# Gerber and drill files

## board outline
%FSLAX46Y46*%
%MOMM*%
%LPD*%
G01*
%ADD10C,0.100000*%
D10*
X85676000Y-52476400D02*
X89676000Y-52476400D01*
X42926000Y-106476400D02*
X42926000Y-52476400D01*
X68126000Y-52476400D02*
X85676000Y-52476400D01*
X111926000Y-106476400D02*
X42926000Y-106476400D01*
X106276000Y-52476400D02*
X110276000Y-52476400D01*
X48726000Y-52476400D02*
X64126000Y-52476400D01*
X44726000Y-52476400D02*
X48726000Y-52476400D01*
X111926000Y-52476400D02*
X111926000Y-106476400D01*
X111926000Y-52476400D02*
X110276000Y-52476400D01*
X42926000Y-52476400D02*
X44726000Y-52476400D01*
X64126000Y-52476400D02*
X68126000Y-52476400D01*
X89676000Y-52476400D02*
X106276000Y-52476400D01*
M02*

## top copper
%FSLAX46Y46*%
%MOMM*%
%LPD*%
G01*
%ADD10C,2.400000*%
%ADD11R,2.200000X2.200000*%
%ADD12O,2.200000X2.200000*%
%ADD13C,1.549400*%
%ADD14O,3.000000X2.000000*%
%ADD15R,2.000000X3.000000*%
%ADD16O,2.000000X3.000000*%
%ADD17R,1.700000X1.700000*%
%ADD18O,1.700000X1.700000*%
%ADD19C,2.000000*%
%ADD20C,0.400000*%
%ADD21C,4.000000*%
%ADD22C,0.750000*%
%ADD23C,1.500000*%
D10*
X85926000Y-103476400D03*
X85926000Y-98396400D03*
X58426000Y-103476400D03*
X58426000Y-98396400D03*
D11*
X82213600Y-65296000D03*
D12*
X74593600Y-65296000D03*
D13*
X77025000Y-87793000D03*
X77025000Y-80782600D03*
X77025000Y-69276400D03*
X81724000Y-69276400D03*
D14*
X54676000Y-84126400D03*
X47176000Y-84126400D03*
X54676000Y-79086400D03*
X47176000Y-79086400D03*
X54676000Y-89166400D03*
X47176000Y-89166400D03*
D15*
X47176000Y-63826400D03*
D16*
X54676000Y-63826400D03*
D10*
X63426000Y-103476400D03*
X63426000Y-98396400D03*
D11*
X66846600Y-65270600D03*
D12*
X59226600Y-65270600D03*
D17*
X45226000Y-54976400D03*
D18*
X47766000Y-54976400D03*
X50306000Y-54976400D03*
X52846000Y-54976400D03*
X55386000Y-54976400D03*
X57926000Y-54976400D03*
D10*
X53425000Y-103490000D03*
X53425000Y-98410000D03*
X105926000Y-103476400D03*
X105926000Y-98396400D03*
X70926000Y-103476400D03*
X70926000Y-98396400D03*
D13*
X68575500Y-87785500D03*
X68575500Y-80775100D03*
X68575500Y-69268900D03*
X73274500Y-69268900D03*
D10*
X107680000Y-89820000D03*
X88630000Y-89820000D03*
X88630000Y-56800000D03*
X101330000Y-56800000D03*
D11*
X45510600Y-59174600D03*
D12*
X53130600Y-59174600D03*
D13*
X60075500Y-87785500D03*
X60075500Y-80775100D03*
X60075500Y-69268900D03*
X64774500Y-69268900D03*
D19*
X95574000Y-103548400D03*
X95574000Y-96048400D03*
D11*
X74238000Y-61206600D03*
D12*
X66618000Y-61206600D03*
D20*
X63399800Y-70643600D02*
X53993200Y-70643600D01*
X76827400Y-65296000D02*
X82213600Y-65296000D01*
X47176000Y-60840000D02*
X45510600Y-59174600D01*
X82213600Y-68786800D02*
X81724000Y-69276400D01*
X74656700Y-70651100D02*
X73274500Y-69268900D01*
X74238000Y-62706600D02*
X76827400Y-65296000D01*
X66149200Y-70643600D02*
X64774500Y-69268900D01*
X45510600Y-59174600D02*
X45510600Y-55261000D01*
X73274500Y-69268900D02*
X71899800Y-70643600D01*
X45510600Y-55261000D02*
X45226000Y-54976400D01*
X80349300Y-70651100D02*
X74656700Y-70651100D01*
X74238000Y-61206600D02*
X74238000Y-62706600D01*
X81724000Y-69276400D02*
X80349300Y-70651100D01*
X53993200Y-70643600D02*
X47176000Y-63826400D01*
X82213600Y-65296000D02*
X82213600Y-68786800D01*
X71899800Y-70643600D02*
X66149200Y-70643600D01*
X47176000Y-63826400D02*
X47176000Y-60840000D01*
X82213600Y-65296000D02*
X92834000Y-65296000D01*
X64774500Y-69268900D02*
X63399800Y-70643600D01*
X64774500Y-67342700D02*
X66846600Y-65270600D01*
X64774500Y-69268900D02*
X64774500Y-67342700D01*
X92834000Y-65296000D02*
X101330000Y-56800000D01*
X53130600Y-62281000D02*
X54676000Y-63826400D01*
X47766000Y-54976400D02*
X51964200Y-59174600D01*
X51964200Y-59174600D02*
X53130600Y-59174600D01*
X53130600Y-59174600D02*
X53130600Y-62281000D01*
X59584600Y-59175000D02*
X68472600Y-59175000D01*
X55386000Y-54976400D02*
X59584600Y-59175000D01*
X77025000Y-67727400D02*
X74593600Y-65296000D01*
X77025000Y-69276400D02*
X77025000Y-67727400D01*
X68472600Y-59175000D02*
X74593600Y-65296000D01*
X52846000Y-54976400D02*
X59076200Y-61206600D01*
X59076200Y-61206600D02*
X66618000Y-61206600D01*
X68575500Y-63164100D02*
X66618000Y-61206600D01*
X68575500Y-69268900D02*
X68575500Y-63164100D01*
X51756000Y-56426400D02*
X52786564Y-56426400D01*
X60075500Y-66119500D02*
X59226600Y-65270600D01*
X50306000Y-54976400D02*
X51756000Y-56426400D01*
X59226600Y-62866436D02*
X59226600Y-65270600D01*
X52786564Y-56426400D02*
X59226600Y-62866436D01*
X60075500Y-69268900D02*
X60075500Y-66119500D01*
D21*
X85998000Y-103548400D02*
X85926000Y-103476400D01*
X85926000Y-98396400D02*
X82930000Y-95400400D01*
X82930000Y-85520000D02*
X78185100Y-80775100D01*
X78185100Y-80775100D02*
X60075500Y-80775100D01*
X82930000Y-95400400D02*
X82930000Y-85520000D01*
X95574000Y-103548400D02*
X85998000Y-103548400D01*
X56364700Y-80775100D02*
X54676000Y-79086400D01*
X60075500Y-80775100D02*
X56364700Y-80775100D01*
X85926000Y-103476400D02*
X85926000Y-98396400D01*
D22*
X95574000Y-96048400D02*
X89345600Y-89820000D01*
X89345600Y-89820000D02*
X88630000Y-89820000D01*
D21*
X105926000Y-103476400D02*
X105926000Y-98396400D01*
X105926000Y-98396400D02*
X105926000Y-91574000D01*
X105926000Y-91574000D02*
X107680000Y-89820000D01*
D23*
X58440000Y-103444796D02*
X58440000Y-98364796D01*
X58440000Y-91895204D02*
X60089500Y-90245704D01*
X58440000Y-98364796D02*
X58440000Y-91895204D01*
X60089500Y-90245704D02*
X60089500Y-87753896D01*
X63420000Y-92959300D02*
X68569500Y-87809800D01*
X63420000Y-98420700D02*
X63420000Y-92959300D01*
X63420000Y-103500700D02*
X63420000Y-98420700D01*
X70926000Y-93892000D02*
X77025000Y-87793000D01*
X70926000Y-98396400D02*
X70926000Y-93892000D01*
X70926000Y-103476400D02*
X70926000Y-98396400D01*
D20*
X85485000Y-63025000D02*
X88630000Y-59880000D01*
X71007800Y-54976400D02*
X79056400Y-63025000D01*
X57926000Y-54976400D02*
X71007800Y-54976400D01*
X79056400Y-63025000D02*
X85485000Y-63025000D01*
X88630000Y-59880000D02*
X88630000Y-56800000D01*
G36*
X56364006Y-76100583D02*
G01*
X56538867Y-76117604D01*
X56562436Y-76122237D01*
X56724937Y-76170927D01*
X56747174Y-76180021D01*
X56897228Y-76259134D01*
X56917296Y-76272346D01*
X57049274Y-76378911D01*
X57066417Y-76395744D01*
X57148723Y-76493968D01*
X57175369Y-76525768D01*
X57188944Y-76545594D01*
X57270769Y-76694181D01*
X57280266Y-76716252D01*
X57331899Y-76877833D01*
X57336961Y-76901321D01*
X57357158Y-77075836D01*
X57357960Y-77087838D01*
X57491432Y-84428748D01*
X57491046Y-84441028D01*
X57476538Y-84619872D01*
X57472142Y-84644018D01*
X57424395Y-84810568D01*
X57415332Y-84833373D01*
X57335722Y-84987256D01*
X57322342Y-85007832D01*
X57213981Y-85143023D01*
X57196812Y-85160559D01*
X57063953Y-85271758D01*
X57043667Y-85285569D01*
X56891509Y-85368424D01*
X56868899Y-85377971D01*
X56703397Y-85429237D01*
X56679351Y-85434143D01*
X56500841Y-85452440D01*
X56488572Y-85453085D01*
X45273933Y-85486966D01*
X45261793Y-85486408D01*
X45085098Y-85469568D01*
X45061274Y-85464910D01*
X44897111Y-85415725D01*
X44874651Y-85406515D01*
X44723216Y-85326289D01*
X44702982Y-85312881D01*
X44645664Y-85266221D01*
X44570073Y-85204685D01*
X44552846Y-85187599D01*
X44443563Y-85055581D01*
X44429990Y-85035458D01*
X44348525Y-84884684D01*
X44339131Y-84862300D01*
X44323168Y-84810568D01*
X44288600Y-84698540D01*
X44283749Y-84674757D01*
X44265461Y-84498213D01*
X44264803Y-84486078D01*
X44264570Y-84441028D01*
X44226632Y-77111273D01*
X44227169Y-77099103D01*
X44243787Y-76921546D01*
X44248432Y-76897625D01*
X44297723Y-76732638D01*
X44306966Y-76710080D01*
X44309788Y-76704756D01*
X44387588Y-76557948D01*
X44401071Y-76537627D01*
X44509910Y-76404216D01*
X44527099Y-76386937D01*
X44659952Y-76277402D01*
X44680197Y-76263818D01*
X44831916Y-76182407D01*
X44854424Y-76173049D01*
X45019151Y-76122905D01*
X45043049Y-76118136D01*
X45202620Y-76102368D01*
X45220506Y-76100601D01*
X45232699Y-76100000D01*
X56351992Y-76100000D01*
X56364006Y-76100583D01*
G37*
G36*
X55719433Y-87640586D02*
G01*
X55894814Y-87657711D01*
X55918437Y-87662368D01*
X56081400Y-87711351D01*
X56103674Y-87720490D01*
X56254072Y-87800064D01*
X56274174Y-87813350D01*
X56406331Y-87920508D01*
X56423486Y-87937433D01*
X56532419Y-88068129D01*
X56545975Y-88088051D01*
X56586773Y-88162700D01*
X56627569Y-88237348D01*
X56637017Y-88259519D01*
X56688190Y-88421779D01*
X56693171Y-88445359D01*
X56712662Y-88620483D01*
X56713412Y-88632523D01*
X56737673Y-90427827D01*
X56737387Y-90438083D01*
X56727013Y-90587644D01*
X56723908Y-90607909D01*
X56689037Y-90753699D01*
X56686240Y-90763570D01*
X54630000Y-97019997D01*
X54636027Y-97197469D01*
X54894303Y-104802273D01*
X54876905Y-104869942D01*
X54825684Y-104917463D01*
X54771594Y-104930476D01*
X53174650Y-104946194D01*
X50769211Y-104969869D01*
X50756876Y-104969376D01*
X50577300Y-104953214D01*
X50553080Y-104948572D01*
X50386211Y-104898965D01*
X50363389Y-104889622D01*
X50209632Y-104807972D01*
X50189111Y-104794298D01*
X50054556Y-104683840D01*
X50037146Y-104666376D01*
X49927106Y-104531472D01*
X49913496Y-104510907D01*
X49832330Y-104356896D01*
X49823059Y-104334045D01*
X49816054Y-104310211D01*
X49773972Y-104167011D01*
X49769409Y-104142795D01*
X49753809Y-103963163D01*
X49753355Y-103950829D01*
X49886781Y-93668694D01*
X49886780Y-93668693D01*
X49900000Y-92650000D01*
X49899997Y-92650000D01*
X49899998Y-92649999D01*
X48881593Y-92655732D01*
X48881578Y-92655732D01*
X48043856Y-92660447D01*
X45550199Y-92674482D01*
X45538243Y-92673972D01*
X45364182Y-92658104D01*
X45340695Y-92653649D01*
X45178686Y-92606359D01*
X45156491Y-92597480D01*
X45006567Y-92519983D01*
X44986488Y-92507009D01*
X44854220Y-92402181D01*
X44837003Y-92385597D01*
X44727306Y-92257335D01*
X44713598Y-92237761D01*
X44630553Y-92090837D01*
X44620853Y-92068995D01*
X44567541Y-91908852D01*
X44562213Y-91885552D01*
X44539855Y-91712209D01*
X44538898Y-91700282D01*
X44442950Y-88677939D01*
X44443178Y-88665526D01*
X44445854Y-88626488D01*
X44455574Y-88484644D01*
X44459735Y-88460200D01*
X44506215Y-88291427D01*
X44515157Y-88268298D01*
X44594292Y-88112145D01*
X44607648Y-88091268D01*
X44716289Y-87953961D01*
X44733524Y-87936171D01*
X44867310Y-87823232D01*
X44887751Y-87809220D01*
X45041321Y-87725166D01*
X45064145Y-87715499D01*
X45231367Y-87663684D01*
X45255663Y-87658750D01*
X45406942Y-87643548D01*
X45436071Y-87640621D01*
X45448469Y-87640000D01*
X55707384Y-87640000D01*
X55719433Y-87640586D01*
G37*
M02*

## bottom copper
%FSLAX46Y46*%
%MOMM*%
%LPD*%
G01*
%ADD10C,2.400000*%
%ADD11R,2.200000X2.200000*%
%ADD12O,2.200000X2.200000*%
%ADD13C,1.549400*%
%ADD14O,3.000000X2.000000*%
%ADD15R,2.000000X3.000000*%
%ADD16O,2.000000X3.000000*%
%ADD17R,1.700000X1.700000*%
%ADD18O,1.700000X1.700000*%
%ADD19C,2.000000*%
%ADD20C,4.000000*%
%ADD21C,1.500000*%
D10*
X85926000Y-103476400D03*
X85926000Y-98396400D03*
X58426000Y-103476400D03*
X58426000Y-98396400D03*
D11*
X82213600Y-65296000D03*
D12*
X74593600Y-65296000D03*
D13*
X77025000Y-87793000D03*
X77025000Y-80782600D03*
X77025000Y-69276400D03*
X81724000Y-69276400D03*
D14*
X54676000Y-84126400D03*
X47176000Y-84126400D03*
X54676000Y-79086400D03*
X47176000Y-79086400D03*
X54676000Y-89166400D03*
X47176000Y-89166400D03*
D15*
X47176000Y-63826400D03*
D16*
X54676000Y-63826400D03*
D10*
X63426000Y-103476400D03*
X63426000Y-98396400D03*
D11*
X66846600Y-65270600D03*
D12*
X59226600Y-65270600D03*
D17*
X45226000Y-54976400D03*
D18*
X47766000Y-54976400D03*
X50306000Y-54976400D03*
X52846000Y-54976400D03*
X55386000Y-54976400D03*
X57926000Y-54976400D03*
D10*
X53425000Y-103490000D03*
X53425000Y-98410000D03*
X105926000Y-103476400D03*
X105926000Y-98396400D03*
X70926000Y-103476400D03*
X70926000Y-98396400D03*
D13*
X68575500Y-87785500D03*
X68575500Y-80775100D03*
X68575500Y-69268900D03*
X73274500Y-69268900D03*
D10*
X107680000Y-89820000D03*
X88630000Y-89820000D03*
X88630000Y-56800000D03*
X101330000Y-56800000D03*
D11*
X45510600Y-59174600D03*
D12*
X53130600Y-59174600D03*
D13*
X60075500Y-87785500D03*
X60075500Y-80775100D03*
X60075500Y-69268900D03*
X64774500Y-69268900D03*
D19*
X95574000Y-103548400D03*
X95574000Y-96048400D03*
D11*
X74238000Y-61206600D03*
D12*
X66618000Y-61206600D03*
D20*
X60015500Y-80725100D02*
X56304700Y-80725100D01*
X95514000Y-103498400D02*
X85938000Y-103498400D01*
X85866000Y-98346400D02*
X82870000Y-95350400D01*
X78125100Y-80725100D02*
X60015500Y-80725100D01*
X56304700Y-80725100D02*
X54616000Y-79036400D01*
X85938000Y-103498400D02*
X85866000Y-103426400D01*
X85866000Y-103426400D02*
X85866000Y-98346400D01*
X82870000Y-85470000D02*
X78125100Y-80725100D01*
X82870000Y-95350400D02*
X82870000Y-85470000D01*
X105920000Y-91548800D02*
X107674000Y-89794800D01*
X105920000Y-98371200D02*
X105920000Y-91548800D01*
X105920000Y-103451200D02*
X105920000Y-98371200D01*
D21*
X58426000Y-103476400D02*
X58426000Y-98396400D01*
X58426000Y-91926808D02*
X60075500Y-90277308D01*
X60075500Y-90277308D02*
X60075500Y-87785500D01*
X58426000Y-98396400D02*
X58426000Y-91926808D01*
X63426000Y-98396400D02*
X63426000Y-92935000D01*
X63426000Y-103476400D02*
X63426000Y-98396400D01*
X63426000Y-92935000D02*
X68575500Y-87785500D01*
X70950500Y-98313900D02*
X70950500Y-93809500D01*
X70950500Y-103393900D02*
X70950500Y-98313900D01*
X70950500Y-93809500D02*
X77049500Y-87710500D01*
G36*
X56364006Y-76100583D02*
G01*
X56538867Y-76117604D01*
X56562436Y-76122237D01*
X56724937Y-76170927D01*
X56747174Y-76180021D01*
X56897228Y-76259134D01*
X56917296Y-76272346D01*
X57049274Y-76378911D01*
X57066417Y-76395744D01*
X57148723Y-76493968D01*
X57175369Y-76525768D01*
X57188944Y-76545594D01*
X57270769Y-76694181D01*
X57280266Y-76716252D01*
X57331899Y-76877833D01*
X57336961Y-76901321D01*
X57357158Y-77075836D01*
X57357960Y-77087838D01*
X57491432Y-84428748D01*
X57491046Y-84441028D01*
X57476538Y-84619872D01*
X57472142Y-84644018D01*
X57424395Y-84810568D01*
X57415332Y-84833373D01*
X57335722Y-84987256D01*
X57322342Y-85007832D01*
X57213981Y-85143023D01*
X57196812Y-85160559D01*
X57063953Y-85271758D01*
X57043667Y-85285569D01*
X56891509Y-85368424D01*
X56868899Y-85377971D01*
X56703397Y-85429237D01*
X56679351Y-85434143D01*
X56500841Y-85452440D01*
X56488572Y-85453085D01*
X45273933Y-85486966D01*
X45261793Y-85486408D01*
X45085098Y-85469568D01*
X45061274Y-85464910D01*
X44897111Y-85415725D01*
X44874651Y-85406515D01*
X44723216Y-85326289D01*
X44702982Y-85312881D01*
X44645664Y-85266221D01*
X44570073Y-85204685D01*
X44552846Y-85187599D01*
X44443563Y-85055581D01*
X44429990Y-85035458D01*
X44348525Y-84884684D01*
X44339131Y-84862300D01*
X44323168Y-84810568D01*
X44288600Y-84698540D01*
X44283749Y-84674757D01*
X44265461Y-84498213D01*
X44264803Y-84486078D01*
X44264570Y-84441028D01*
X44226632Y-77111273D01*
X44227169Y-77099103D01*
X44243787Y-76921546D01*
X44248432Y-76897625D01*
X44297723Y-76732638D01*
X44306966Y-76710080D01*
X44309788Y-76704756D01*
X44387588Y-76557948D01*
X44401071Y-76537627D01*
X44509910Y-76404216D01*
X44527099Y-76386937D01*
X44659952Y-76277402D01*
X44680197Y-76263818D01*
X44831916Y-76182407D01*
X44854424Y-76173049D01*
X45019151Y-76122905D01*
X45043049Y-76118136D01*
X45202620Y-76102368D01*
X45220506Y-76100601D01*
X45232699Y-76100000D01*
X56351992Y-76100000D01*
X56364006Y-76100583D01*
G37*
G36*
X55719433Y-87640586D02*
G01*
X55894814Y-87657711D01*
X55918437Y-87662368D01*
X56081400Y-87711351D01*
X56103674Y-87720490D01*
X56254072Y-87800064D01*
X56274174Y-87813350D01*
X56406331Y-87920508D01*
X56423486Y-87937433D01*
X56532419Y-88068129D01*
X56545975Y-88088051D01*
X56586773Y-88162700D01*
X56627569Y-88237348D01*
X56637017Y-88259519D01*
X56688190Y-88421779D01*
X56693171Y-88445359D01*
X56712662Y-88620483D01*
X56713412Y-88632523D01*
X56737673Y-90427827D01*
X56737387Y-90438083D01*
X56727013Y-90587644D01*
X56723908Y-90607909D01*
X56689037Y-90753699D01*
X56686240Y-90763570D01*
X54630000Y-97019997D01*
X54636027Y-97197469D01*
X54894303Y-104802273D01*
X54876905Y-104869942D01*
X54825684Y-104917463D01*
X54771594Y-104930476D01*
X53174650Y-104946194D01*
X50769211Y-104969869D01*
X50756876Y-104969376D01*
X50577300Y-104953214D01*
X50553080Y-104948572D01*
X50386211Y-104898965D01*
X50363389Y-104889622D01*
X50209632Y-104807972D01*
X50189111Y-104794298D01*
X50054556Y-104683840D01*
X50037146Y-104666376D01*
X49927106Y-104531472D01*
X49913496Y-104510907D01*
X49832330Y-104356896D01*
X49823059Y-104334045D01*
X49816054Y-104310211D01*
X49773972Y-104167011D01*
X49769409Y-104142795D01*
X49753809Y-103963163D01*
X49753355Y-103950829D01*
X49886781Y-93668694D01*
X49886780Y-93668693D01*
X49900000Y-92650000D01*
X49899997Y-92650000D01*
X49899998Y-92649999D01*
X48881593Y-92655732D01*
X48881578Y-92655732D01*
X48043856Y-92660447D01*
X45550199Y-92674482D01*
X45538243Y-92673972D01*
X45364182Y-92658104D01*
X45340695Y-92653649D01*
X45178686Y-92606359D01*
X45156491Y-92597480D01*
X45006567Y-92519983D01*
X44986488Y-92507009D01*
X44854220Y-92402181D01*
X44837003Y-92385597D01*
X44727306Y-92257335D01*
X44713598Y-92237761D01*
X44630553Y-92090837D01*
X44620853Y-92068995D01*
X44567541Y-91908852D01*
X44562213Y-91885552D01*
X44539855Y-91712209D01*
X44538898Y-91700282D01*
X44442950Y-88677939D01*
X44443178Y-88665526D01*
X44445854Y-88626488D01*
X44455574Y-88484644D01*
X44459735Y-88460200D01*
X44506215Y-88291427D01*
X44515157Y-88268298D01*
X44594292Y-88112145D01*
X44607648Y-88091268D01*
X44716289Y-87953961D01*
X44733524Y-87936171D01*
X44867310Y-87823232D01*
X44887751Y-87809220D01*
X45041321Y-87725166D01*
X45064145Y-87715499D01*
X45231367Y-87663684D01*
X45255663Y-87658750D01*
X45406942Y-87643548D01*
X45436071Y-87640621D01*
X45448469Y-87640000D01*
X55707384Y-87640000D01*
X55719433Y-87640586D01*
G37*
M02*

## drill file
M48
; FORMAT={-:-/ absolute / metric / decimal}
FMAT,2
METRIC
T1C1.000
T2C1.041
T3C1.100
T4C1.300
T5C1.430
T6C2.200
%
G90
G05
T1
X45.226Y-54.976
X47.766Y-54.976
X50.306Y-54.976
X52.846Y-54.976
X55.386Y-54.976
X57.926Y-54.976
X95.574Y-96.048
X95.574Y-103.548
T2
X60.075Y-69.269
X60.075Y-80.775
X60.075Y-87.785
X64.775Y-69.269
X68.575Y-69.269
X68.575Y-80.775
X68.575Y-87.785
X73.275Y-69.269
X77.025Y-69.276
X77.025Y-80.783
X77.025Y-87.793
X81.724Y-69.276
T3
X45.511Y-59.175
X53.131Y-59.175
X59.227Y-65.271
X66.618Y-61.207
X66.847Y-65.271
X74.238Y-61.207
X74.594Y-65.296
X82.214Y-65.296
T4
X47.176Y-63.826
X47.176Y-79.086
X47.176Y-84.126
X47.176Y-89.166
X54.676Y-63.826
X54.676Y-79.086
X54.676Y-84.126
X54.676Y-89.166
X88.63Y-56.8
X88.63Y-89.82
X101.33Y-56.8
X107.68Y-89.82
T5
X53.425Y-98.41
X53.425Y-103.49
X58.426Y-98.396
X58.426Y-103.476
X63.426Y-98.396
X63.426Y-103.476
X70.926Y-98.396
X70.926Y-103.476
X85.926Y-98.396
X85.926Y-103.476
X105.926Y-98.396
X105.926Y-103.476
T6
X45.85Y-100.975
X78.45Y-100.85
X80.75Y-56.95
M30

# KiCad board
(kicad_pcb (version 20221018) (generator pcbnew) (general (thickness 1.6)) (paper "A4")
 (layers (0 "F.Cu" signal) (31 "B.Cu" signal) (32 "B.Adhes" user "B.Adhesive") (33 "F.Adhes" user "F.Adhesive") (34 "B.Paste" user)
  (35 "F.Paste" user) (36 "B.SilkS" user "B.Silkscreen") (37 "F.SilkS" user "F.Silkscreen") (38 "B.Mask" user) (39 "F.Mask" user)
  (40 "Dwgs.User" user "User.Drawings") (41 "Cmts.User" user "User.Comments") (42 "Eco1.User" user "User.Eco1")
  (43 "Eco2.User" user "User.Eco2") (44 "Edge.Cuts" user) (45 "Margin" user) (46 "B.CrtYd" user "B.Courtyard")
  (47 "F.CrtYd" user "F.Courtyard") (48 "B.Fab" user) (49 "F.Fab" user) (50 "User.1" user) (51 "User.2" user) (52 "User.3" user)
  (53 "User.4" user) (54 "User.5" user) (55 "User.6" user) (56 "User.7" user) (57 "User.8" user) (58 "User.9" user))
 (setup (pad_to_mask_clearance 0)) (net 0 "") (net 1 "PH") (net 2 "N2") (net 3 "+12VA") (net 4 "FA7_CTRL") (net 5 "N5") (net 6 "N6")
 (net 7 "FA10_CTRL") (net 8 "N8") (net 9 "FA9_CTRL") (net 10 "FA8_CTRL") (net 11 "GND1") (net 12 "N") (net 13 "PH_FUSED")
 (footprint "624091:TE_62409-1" (layer "F.Cu") (at 85.926 100.9364 90)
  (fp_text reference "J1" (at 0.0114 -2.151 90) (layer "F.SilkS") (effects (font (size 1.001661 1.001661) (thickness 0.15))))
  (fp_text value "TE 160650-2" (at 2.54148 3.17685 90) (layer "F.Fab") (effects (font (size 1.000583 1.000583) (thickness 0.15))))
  (pad "1" thru_hole circle (at -2.54 0 90) (size 2.4 2.4) (drill 1.43) (layers "*.Cu" "*.Mask") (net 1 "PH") (solder_mask_margin 0.102))
  (pad "1" thru_hole circle (at 2.54 0 90) (size 2.4 2.4) (drill 1.43) (layers "*.Cu" "*.Mask") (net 1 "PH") (solder_mask_margin 0.102)))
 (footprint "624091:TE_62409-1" (layer "F.Cu") (at 58.426 100.9364 90)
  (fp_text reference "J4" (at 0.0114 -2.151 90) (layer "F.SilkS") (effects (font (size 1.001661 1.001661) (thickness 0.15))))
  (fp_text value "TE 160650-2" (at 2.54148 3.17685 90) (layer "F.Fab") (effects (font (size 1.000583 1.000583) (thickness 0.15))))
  (pad "1" thru_hole circle (at -2.54 0 90) (size 2.4 2.4) (drill 1.43) (layers "*.Cu" "*.Mask") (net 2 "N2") (solder_mask_margin 0.102))
  (pad "1" thru_hole circle (at 2.54 0 90) (size 2.4 2.4) (drill 1.43) (layers "*.Cu" "*.Mask") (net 2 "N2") (solder_mask_margin 0.102)))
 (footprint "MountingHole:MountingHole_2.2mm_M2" (layer "F.Cu") (at 80.75 56.95)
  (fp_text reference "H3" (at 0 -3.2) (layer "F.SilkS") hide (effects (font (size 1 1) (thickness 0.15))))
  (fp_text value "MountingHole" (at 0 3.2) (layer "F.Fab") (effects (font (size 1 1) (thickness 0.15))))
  (pad "" np_thru_hole circle (at 0 0) (size 2.2 2.2) (drill 2.2) (layers "F&B.Cu" "*.Mask")))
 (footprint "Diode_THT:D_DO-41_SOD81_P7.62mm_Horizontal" (layer "F.Cu") (at 82.2136 65.296 180)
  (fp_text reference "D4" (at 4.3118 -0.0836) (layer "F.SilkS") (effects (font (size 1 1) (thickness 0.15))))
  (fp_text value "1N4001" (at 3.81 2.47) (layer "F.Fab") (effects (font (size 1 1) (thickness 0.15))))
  (pad "1" thru_hole rect (at 0 0 180) (size 2.2 2.2) (drill 1.1) (layers "*.Cu" "*.Mask") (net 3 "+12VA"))
  (pad "2" thru_hole oval (at 7.62 0 180) (size 2.2 2.2) (drill 1.1) (layers "*.Cu" "*.Mask") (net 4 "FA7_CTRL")))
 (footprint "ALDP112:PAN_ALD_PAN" (layer "F.Cu") (at 81.725 87.793 180)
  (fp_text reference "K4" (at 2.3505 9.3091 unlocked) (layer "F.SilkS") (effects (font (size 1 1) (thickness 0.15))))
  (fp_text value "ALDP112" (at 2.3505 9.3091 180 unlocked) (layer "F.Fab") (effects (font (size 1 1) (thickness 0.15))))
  (pad "1" thru_hole circle (at 4.7 0 180) (size 1.5494 1.5494) (drill 1.0414) (layers "*.Cu" "*.Mask") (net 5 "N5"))
  (pad "2" thru_hole circle (at 4.7 7.0104 180) (size 1.5494 1.5494) (drill 1.0414) (layers "*.Cu" "*.Mask") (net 1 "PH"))
  (pad "3" thru_hole circle (at 4.7 18.5166 180) (size 1.5494 1.5494) (drill 1.0414) (layers "*.Cu" "*.Mask") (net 4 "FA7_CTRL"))
  (pad "4" thru_hole circle (at 0.001 18.5166 180) (size 1.5494 1.5494) (drill 1.0414) (layers "*.Cu" "*.Mask") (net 3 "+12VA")))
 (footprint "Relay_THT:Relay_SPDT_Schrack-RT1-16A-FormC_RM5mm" (layer "F.Cu") (at 47.176 63.8264 -90)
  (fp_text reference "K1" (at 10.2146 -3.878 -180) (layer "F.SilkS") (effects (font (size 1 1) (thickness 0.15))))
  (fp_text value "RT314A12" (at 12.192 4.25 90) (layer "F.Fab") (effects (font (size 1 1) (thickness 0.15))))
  (pad "11" thru_hole oval (at 20.3 -7.5 90) (size 2 3) (drill 1.3) (layers "*.Cu" "*.Mask") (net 1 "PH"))
  (pad "11" thru_hole oval (at 20.3 0 90) (size 2 3) (drill 1.3) (layers "*.Cu" "*.Mask") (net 1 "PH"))
  (pad "12" thru_hole oval (at 15.26 -7.5 90) (size 2 3) (drill 1.3) (layers "*.Cu" "*.Mask") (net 1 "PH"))
  (pad "12" thru_hole oval (at 15.26 0 90) (size 2 3) (drill 1.3) (layers "*.Cu" "*.Mask") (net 1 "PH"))
  (pad "14" thru_hole oval (at 25.34 -7.5 90) (size 2 3) (drill 1.3) (layers "*.Cu" "*.Mask") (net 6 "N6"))
  (pad "14" thru_hole oval (at 25.34 0 90) (size 2 3) (drill 1.3) (layers "*.Cu" "*.Mask") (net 6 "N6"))
  (pad "A1" thru_hole rect (at 0 0 90) (size 3 2) (drill 1.3) (layers "*.Cu" "*.Mask") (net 3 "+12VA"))
  (pad "A2" thru_hole oval (at 0 -7.5 90) (size 3 2) (drill 1.3) (layers "*.Cu" "*.Mask") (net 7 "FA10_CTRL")))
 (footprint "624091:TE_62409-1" (layer "F.Cu") (at 63.426 100.9364 90)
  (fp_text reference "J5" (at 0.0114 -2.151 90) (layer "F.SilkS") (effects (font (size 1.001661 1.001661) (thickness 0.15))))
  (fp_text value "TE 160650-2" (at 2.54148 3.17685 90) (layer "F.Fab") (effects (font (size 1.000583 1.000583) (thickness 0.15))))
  (pad "1" thru_hole circle (at -2.54 0 90) (size 2.4 2.4) (drill 1.43) (layers "*.Cu" "*.Mask") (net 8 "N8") (solder_mask_margin 0.102))
  (pad "1" thru_hole circle (at 2.54 0 90) (size 2.4 2.4) (drill 1.43) (layers "*.Cu" "*.Mask") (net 8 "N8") (solder_mask_margin 0.102)))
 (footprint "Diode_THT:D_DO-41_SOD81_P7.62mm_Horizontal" (layer "F.Cu") (at 66.8466 65.2706 180)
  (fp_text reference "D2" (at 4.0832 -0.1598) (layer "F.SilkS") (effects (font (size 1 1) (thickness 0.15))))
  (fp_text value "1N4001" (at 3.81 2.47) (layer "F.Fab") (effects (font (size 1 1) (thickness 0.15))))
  (pad "1" thru_hole rect (at 0 0 180) (size 2.2 2.2) (drill 1.1) (layers "*.Cu" "*.Mask") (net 3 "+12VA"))
  (pad "2" thru_hole oval (at 7.62 0 180) (size 2.2 2.2) (drill 1.1) (layers "*.Cu" "*.Mask") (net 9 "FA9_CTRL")))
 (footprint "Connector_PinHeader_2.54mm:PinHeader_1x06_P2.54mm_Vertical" (layer "F.Cu") (at 45.226 54.9764 90)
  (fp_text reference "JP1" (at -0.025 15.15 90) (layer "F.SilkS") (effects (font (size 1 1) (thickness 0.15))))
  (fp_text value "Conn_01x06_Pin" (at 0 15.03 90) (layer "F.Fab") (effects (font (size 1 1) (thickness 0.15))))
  (pad "1" thru_hole rect (at 0 0 90) (size 1.7 1.7) (drill 1) (layers "*.Cu" "*.Mask") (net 3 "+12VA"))
  (pad "2" thru_hole oval (at 0 2.54 90) (size 1.7 1.7) (drill 1) (layers "*.Cu" "*.Mask") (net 7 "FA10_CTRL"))
  (pad "3" thru_hole oval (at 0 5.08 90) (size 1.7 1.7) (drill 1) (layers "*.Cu" "*.Mask") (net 9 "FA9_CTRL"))
  (pad "4" thru_hole oval (at 0 7.62 90) (size 1.7 1.7) (drill 1) (layers "*.Cu" "*.Mask") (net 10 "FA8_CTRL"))
  (pad "5" thru_hole oval (at 0 10.16 90) (size 1.7 1.7) (drill 1) (layers "*.Cu" "*.Mask") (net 4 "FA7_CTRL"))
  (pad "6" thru_hole oval (at 0 12.7 90) (size 1.7 1.7) (drill 1) (layers "*.Cu" "*.Mask") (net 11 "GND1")))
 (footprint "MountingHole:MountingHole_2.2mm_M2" (layer "F.Cu") (at 45.85 100.975)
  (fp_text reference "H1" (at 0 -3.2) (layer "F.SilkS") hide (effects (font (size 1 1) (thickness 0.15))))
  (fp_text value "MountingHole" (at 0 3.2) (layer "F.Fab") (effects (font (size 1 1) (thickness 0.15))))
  (pad "" np_thru_hole circle (at 0 0) (size 2.2 2.2) (drill 2.2) (layers "*.Cu" "*.Mask")))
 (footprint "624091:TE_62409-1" (layer "F.Cu") (at 53.425 100.95 90)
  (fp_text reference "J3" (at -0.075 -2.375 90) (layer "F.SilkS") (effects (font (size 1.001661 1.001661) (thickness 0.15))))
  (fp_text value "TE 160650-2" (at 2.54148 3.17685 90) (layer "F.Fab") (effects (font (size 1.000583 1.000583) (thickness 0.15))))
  (pad "1" thru_hole circle (at -2.54 0 90) (size 2.4 2.4) (drill 1.43) (layers "*.Cu" "*.Mask") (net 6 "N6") (solder_mask_margin 0.102))
  (pad "1" thru_hole circle (at 2.54 0 90) (size 2.4 2.4) (drill 1.43) (layers "*.Cu" "*.Mask") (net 6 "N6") (solder_mask_margin 0.102)))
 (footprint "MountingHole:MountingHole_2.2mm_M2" (layer "F.Cu") (at 78.45 100.85)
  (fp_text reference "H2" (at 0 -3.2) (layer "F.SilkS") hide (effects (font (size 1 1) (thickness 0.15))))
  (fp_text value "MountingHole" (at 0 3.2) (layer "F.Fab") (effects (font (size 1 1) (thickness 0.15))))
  (pad "" np_thru_hole circle (at 0 0) (size 2.2 2.2) (drill 2.2) (layers "F&B.Cu" "*.Mask")))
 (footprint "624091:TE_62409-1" (layer "F.Cu") (at 105.926 100.9364 90)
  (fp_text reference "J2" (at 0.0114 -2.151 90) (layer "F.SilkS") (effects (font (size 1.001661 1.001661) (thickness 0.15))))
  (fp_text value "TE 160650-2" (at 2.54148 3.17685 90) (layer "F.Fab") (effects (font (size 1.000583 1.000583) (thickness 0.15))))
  (pad "1" thru_hole circle (at -2.54 0 90) (size 2.4 2.4) (drill 1.43) (layers "*.Cu" "*.Mask") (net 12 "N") (solder_mask_margin 0.102))
  (pad "1" thru_hole circle (at 2.54 0 90) (size 2.4 2.4) (drill 1.43) (layers "*.Cu" "*.Mask") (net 12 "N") (solder_mask_margin 0.102)))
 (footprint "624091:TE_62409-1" (layer "F.Cu") (at 70.926 100.9364 90)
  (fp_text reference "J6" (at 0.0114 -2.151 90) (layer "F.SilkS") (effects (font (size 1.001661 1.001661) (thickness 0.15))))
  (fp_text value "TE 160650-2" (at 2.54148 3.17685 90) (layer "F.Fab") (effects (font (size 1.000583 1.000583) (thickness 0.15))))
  (pad "1" thru_hole circle (at -2.54 0 90) (size 2.4 2.4) (drill 1.43) (layers "*.Cu" "*.Mask") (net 5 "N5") (solder_mask_margin 0.102))
  (pad "1" thru_hole circle (at 2.54 0 90) (size 2.4 2.4) (drill 1.43) (layers "*.Cu" "*.Mask") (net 5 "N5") (solder_mask_margin 0.102)))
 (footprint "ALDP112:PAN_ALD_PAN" (layer "F.Cu") (at 73.2755 87.7855 180)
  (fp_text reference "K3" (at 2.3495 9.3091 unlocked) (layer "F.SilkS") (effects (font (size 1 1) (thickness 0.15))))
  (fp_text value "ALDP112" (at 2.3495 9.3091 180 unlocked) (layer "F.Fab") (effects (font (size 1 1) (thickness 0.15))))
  (pad "1" thru_hole circle (at 4.7 0 180) (size 1.5494 1.5494) (drill 1.0414) (layers "*.Cu" "*.Mask") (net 8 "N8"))
  (pad "2" thru_hole circle (at 4.7 7.0104 180) (size 1.5494 1.5494) (drill 1.0414) (layers "*.Cu" "*.Mask") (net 1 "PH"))
  (pad "3" thru_hole circle (at 4.7 18.5166 180) (size 1.5494 1.5494) (drill 1.0414) (layers "*.Cu" "*.Mask") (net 10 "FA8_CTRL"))
  (pad "4" thru_hole circle (at 0.001 18.5166 180) (size 1.5494 1.5494) (drill 1.0414) (layers "*.Cu" "*.Mask") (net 3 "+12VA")))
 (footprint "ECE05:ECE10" (layer "F.Cu") (at 111.49 54.26 180)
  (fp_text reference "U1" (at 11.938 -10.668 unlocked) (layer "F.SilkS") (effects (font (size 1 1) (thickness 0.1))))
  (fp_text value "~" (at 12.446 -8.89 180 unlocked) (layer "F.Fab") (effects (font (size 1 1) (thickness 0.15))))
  (pad "1" thru_hole circle (at 3.81 -35.56 180) (size 2.4 2.4) (drill 1.3) (layers "*.Cu" "*.Mask") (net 12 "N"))
  (pad "2" thru_hole circle (at 22.86 -35.56 180) (size 2.4 2.4) (drill 1.3) (layers "*.Cu" "*.Mask") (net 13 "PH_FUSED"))
  (pad "3" thru_hole circle (at 22.86 -2.54 180) (size 2.4 2.4) (drill 1.3) (layers "*.Cu" "*.Mask") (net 11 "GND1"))
  (pad "4" thru_hole circle (at 10.16 -2.54 180) (size 2.4 2.4) (drill 1.3) (layers "*.Cu" "*.Mask") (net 3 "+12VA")))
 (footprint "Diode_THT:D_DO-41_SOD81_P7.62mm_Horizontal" (layer "F.Cu") (at 45.5106 59.1746)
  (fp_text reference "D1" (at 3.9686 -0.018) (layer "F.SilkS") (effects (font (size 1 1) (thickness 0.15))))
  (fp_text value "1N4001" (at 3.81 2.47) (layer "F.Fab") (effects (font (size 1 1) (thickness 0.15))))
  (pad "1" thru_hole rect (at 0 0) (size 2.2 2.2) (drill 1.1) (layers "*.Cu" "*.Mask") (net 3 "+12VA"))
  (pad "2" thru_hole oval (at 7.62 0) (size 2.2 2.2) (drill 1.1) (layers "*.Cu" "*.Mask") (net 7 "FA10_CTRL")))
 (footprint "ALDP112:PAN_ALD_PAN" (layer "F.Cu") (at 64.7755 87.7855 180)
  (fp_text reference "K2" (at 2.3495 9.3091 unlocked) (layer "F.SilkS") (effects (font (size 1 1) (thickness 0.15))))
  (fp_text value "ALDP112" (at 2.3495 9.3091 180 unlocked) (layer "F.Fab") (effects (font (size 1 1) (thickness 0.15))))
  (pad "1" thru_hole circle (at 4.7 0 180) (size 1.5494 1.5494) (drill 1.0414) (layers "*.Cu" "*.Mask") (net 2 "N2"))
  (pad "2" thru_hole circle (at 4.7 7.0104 180) (size 1.5494 1.5494) (drill 1.0414) (layers "*.Cu" "*.Mask") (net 1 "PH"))
  (pad "3" thru_hole circle (at 4.7 18.5166 180) (size 1.5494 1.5494) (drill 1.0414) (layers "*.Cu" "*.Mask") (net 9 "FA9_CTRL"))
  (pad "4" thru_hole circle (at 0.001 18.5166 180) (size 1.5494 1.5494) (drill 1.0414) (layers "*.Cu" "*.Mask") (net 3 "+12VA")))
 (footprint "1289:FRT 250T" (layer "F.Cu") (at 98.074 105.5484 90)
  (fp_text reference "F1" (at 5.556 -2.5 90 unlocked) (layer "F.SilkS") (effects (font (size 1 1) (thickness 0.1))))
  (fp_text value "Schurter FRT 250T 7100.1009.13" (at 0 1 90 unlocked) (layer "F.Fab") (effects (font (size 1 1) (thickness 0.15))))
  (pad "1" thru_hole circle (at 2 -2.5 90) (size 2 2) (drill 1) (layers "*.Cu" "*.Mask") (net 1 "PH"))
  (pad "2" thru_hole circle (at 9.5 -2.5 90) (size 2 2) (drill 1) (layers "*.Cu" "*.Mask") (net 13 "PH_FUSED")))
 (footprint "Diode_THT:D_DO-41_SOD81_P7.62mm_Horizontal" (layer "F.Cu") (at 74.238 61.2066 180)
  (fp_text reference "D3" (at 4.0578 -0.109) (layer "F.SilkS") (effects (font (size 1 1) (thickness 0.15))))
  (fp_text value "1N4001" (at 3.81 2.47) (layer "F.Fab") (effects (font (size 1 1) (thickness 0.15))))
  (pad "1" thru_hole rect (at 0 0 180) (size 2.2 2.2) (drill 1.1) (layers "*.Cu" "*.Mask") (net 3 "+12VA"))
  (pad "2" thru_hole oval (at 7.62 0 180) (size 2.2 2.2) (drill 1.1) (layers "*.Cu" "*.Mask") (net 10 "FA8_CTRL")))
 (gr_line (start 85.676 52.4764) (end 89.676 52.4764) (stroke (width 0.1) (type default)) (layer "Edge.Cuts"))
 (gr_line (start 42.926 106.4764) (end 42.926 52.4764) (stroke (width 0.1) (type default)) (layer "Edge.Cuts"))
 (gr_line (start 68.126 52.4764) (end 85.676 52.4764) (stroke (width 0.1) (type default)) (layer "Edge.Cuts"))
 (gr_line (start 111.926 106.4764) (end 42.926 106.4764) (stroke (width 0.1) (type default)) (layer "Edge.Cuts"))
 (gr_line (start 106.276 52.4764) (end 110.276 52.4764) (stroke (width 0.1) (type default)) (layer "Edge.Cuts"))
 (gr_line (start 48.726 52.4764) (end 64.126 52.4764) (stroke (width 0.1) (type default)) (layer "Edge.Cuts"))
 (gr_line (start 44.726 52.4764) (end 48.726 52.4764) (stroke (width 0.1) (type default)) (layer "Edge.Cuts"))
 (gr_line (start 111.926 52.4764) (end 111.926 106.4764) (stroke (width 0.1) (type default)) (layer "Edge.Cuts"))
 (gr_line (start 111.926 52.4764) (end 110.276 52.4764) (stroke (width 0.1) (type default)) (layer "Edge.Cuts"))
 (gr_line (start 42.926 52.4764) (end 44.726 52.4764) (stroke (width 0.1) (type default)) (layer "Edge.Cuts"))
 (gr_line (start 64.126 52.4764) (end 68.126 52.4764) (stroke (width 0.1) (type default)) (layer "Edge.Cuts"))
 (gr_line (start 89.676 52.4764) (end 106.276 52.4764) (stroke (width 0.1) (type default)) (layer "Edge.Cuts"))
 (segment (start 63.3998 70.6436) (end 53.9932 70.6436) (width 0.4) (layer "F.Cu") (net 3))
 (segment (start 76.8274 65.296) (end 82.2136 65.296) (width 0.4) (layer "F.Cu") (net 3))
 (segment (start 47.176 60.84) (end 45.5106 59.1746) (width 0.4) (layer "F.Cu") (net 3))
 (segment (start 82.2136 68.7868) (end 81.724 69.2764) (width 0.4) (layer "F.Cu") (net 3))
 (segment (start 74.6567 70.6511) (end 73.2745 69.2689) (width 0.4) (layer "F.Cu") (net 3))
 (segment (start 74.238 62.7066) (end 76.8274 65.296) (width 0.4) (layer "F.Cu") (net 3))
 (segment (start 66.1492 70.6436) (end 64.7745 69.2689) (width 0.4) (layer "F.Cu") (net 3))
 (segment (start 45.5106 59.1746) (end 45.5106 55.261) (width 0.4) (layer "F.Cu") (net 3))
 (segment (start 73.2745 69.2689) (end 71.8998 70.6436) (width 0.4) (layer "F.Cu") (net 3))
 (segment (start 45.5106 55.261) (end 45.226 54.9764) (width 0.4) (layer "F.Cu") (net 3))
 (segment (start 80.3493 70.6511) (end 74.6567 70.6511) (width 0.4) (layer "F.Cu") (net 3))
 (segment (start 74.238 61.2066) (end 74.238 62.7066) (width 0.4) (layer "F.Cu") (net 3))
 (segment (start 81.724 69.2764) (end 80.3493 70.6511) (width 0.4) (layer "F.Cu") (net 3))
 (segment (start 53.9932 70.6436) (end 47.176 63.8264) (width 0.4) (layer "F.Cu") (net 3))
 (segment (start 82.2136 65.296) (end 82.2136 68.7868) (width 0.4) (layer "F.Cu") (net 3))
 (segment (start 71.8998 70.6436) (end 66.1492 70.6436) (width 0.4) (layer "F.Cu") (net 3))
 (segment (start 47.176 63.8264) (end 47.176 60.84) (width 0.4) (layer "F.Cu") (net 3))
 (segment (start 82.2136 65.296) (end 92.834 65.296) (width 0.4) (layer "F.Cu") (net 3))
 (segment (start 64.7745 69.2689) (end 63.3998 70.6436) (width 0.4) (layer "F.Cu") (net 3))
 (segment (start 64.7745 67.3427) (end 66.8466 65.2706) (width 0.4) (layer "F.Cu") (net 3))
 (segment (start 64.7745 69.2689) (end 64.7745 67.3427) (width 0.4) (layer "F.Cu") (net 3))
 (segment (start 92.834 65.296) (end 101.33 56.8) (width 0.4) (layer "F.Cu") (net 3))
 (segment (start 53.1306 62.281) (end 54.676 63.8264) (width 0.4) (layer "F.Cu") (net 7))
 (segment (start 47.766 54.9764) (end 51.9642 59.1746) (width 0.4) (layer "F.Cu") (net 7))
 (segment (start 51.9642 59.1746) (end 53.1306 59.1746) (width 0.4) (layer "F.Cu") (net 7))
 (segment (start 53.1306 59.1746) (end 53.1306 62.281) (width 0.4) (layer "F.Cu") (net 7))
 (segment (start 59.5846 59.175) (end 68.4726 59.175) (width 0.4) (layer "F.Cu") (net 4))
 (segment (start 55.386 54.9764) (end 59.5846 59.175) (width 0.4) (layer "F.Cu") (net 4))
 (segment (start 77.025 67.7274) (end 74.5936 65.296) (width 0.4) (layer "F.Cu") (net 4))
 (segment (start 77.025 69.2764) (end 77.025 67.7274) (width 0.4) (layer "F.Cu") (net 4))
 (segment (start 68.4726 59.175) (end 74.5936 65.296) (width 0.4) (layer "F.Cu") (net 4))
 (segment (start 52.846 54.9764) (end 59.0762 61.2066) (width 0.4) (layer "F.Cu") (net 10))
 (segment (start 59.0762 61.2066) (end 66.618 61.2066) (width 0.4) (layer "F.Cu") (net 10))
 (segment (start 68.5755 63.1641) (end 66.618 61.2066) (width 0.4) (layer "F.Cu") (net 10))
 (segment (start 68.5755 69.2689) (end 68.5755 63.1641) (width 0.4) (layer "F.Cu") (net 10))
 (segment (start 51.756 56.4264) (end 52.786564 56.4264) (width 0.4) (layer "F.Cu") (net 9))
 (segment (start 60.0755 66.1195) (end 59.2266 65.2706) (width 0.4) (layer "F.Cu") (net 9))
 (segment (start 50.306 54.9764) (end 51.756 56.4264) (width 0.4) (layer "F.Cu") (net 9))
 (segment (start 59.2266 62.866436) (end 59.2266 65.2706) (width 0.4) (layer "F.Cu") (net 9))
 (segment (start 52.786564 56.4264) (end 59.2266 62.866436) (width 0.4) (layer "F.Cu") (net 9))
 (segment (start 60.0755 69.2689) (end 60.0755 66.1195) (width 0.4) (layer "F.Cu") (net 9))
 (segment (start 85.998 103.5484) (end 85.926 103.4764) (width 4) (layer "F.Cu") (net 1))
 (segment (start 85.926 98.3964) (end 82.93 95.4004) (width 4) (layer "F.Cu") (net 1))
 (segment (start 82.93 85.52) (end 78.1851 80.7751) (width 4) (layer "F.Cu") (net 1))
 (segment (start 78.1851 80.7751) (end 60.0755 80.7751) (width 4) (layer "F.Cu") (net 1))
 (segment (start 82.93 95.4004) (end 82.93 85.52) (width 4) (layer "F.Cu") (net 1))
 (segment (start 95.574 103.5484) (end 85.998 103.5484) (width 4) (layer "F.Cu") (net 1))
 (segment (start 56.3647 80.7751) (end 54.676 79.0864) (width 4) (layer "F.Cu") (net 1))
 (segment (start 60.0755 80.7751) (end 56.3647 80.7751) (width 4) (layer "F.Cu") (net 1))
 (segment (start 85.926 103.4764) (end 85.926 98.3964) (width 4) (layer "F.Cu") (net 1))
 (segment (start 60.0155 80.7251) (end 56.3047 80.7251) (width 4) (layer "B.Cu") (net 1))
 (segment (start 95.514 103.4984) (end 85.938 103.4984) (width 4) (layer "B.Cu") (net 1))
 (segment (start 85.866 98.3464) (end 82.87 95.3504) (width 4) (layer "B.Cu") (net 1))
 (segment (start 78.1251 80.7251) (end 60.0155 80.7251) (width 4) (layer "B.Cu") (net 1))
 (segment (start 56.3047 80.7251) (end 54.616 79.0364) (width 4) (layer "B.Cu") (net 1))
 (segment (start 85.938 103.4984) (end 85.866 103.4264) (width 4) (layer "B.Cu") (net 1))
 (segment (start 85.866 103.4264) (end 85.866 98.3464) (width 4) (layer "B.Cu") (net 1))
 (segment (start 82.87 85.47) (end 78.1251 80.7251) (width 4) (layer "B.Cu") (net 1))
 (segment (start 82.87 95.3504) (end 82.87 85.47) (width 4) (layer "B.Cu") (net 1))
 (segment (start 95.574 96.0484) (end 89.3456 89.82) (width 0.75) (layer "F.Cu") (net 13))
 (segment (start 89.3456 89.82) (end 88.63 89.82) (width 0.75) (layer "F.Cu") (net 13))
 (segment (start 105.926 103.4764) (end 105.926 98.3964) (width 4) (layer "F.Cu") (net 12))
 (segment (start 105.926 98.3964) (end 105.926 91.574) (width 4) (layer "F.Cu") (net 12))
 (segment (start 105.926 91.574) (end 107.68 89.82) (width 4) (layer "F.Cu") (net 12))
 (segment (start 105.92 91.5488) (end 107.674 89.7948) (width 4) (layer "B.Cu") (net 12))
 (segment (start 105.92 98.3712) (end 105.92 91.5488) (width 4) (layer "B.Cu") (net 12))
 (segment (start 105.92 103.4512) (end 105.92 98.3712) (width 4) (layer "B.Cu") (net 12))
 (segment (start 58.44 103.444796) (end 58.44 98.364796) (width 1.5) (layer "F.Cu") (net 2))
 (segment (start 58.44 91.895204) (end 60.0895 90.245704) (width 1.5) (layer "F.Cu") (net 2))
 (segment (start 58.44 98.364796) (end 58.44 91.895204) (width 1.5) (layer "F.Cu") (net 2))
 (segment (start 60.0895 90.245704) (end 60.0895 87.753896) (width 1.5) (layer "F.Cu") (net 2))
 (segment (start 58.426 103.4764) (end 58.426 98.3964) (width 1.5) (layer "B.Cu") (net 2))
 (segment (start 58.426 91.926808) (end 60.0755 90.277308) (width 1.5) (layer "B.Cu") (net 2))
 (segment (start 60.0755 90.277308) (end 60.0755 87.7855) (width 1.5) (layer "B.Cu") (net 2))
 (segment (start 58.426 98.3964) (end 58.426 91.926808) (width 1.5) (layer "B.Cu") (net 2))
 (segment (start 63.42 92.9593) (end 68.5695 87.8098) (width 1.5) (layer "F.Cu") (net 8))
 (segment (start 63.42 98.4207) (end 63.42 92.9593) (width 1.5) (layer "F.Cu") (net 8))
 (segment (start 63.42 103.5007) (end 63.42 98.4207) (width 1.5) (layer "F.Cu") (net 8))
 (segment (start 63.426 98.3964) (end 63.426 92.935) (width 1.5) (layer "B.Cu") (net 8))
 (segment (start 63.426 103.4764) (end 63.426 98.3964) (width 1.5) (layer "B.Cu") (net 8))
 (segment (start 63.426 92.935) (end 68.5755 87.7855) (width 1.5) (layer "B.Cu") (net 8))
 (segment (start 70.926 93.892) (end 77.025 87.793) (width 1.5) (layer "F.Cu") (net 5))
 (segment (start 70.926 98.3964) (end 70.926 93.892) (width 1.5) (layer "F.Cu") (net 5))
 (segment (start 70.926 103.4764) (end 70.926 98.3964) (width 1.5) (layer "F.Cu") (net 5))
 (segment (start 70.9505 98.3139) (end 70.9505 93.8095) (width 1.5) (layer "B.Cu") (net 5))
 (segment (start 70.9505 103.3939) (end 70.9505 98.3139) (width 1.5) (layer "B.Cu") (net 5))
 (segment (start 70.9505 93.8095) (end 77.0495 87.7105) (width 1.5) (layer "B.Cu") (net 5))
 (segment (start 85.485 63.025) (end 88.63 59.88) (width 0.4) (layer "F.Cu") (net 11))
 (segment (start 71.0078 54.9764) (end 79.0564 63.025) (width 0.4) (layer "F.Cu") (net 11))
 (segment (start 57.926 54.9764) (end 71.0078 54.9764) (width 0.4) (layer "F.Cu") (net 11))
 (segment (start 79.0564 63.025) (end 85.485 63.025) (width 0.4) (layer "F.Cu") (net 11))
 (segment (start 88.63 59.88) (end 88.63 56.8) (width 0.4) (layer "F.Cu") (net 11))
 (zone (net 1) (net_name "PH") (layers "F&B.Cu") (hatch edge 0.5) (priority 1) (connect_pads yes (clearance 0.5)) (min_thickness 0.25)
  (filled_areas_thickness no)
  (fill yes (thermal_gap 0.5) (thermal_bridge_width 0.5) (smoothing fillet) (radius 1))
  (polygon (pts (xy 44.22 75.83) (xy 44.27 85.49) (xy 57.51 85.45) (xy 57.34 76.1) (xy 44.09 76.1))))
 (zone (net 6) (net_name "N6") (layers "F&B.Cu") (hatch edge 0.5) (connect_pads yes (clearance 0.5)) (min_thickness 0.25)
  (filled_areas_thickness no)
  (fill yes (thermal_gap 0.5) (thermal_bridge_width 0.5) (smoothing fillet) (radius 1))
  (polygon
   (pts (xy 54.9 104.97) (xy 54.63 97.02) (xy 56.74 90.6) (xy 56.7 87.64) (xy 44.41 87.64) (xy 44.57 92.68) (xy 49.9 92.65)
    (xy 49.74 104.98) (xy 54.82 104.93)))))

